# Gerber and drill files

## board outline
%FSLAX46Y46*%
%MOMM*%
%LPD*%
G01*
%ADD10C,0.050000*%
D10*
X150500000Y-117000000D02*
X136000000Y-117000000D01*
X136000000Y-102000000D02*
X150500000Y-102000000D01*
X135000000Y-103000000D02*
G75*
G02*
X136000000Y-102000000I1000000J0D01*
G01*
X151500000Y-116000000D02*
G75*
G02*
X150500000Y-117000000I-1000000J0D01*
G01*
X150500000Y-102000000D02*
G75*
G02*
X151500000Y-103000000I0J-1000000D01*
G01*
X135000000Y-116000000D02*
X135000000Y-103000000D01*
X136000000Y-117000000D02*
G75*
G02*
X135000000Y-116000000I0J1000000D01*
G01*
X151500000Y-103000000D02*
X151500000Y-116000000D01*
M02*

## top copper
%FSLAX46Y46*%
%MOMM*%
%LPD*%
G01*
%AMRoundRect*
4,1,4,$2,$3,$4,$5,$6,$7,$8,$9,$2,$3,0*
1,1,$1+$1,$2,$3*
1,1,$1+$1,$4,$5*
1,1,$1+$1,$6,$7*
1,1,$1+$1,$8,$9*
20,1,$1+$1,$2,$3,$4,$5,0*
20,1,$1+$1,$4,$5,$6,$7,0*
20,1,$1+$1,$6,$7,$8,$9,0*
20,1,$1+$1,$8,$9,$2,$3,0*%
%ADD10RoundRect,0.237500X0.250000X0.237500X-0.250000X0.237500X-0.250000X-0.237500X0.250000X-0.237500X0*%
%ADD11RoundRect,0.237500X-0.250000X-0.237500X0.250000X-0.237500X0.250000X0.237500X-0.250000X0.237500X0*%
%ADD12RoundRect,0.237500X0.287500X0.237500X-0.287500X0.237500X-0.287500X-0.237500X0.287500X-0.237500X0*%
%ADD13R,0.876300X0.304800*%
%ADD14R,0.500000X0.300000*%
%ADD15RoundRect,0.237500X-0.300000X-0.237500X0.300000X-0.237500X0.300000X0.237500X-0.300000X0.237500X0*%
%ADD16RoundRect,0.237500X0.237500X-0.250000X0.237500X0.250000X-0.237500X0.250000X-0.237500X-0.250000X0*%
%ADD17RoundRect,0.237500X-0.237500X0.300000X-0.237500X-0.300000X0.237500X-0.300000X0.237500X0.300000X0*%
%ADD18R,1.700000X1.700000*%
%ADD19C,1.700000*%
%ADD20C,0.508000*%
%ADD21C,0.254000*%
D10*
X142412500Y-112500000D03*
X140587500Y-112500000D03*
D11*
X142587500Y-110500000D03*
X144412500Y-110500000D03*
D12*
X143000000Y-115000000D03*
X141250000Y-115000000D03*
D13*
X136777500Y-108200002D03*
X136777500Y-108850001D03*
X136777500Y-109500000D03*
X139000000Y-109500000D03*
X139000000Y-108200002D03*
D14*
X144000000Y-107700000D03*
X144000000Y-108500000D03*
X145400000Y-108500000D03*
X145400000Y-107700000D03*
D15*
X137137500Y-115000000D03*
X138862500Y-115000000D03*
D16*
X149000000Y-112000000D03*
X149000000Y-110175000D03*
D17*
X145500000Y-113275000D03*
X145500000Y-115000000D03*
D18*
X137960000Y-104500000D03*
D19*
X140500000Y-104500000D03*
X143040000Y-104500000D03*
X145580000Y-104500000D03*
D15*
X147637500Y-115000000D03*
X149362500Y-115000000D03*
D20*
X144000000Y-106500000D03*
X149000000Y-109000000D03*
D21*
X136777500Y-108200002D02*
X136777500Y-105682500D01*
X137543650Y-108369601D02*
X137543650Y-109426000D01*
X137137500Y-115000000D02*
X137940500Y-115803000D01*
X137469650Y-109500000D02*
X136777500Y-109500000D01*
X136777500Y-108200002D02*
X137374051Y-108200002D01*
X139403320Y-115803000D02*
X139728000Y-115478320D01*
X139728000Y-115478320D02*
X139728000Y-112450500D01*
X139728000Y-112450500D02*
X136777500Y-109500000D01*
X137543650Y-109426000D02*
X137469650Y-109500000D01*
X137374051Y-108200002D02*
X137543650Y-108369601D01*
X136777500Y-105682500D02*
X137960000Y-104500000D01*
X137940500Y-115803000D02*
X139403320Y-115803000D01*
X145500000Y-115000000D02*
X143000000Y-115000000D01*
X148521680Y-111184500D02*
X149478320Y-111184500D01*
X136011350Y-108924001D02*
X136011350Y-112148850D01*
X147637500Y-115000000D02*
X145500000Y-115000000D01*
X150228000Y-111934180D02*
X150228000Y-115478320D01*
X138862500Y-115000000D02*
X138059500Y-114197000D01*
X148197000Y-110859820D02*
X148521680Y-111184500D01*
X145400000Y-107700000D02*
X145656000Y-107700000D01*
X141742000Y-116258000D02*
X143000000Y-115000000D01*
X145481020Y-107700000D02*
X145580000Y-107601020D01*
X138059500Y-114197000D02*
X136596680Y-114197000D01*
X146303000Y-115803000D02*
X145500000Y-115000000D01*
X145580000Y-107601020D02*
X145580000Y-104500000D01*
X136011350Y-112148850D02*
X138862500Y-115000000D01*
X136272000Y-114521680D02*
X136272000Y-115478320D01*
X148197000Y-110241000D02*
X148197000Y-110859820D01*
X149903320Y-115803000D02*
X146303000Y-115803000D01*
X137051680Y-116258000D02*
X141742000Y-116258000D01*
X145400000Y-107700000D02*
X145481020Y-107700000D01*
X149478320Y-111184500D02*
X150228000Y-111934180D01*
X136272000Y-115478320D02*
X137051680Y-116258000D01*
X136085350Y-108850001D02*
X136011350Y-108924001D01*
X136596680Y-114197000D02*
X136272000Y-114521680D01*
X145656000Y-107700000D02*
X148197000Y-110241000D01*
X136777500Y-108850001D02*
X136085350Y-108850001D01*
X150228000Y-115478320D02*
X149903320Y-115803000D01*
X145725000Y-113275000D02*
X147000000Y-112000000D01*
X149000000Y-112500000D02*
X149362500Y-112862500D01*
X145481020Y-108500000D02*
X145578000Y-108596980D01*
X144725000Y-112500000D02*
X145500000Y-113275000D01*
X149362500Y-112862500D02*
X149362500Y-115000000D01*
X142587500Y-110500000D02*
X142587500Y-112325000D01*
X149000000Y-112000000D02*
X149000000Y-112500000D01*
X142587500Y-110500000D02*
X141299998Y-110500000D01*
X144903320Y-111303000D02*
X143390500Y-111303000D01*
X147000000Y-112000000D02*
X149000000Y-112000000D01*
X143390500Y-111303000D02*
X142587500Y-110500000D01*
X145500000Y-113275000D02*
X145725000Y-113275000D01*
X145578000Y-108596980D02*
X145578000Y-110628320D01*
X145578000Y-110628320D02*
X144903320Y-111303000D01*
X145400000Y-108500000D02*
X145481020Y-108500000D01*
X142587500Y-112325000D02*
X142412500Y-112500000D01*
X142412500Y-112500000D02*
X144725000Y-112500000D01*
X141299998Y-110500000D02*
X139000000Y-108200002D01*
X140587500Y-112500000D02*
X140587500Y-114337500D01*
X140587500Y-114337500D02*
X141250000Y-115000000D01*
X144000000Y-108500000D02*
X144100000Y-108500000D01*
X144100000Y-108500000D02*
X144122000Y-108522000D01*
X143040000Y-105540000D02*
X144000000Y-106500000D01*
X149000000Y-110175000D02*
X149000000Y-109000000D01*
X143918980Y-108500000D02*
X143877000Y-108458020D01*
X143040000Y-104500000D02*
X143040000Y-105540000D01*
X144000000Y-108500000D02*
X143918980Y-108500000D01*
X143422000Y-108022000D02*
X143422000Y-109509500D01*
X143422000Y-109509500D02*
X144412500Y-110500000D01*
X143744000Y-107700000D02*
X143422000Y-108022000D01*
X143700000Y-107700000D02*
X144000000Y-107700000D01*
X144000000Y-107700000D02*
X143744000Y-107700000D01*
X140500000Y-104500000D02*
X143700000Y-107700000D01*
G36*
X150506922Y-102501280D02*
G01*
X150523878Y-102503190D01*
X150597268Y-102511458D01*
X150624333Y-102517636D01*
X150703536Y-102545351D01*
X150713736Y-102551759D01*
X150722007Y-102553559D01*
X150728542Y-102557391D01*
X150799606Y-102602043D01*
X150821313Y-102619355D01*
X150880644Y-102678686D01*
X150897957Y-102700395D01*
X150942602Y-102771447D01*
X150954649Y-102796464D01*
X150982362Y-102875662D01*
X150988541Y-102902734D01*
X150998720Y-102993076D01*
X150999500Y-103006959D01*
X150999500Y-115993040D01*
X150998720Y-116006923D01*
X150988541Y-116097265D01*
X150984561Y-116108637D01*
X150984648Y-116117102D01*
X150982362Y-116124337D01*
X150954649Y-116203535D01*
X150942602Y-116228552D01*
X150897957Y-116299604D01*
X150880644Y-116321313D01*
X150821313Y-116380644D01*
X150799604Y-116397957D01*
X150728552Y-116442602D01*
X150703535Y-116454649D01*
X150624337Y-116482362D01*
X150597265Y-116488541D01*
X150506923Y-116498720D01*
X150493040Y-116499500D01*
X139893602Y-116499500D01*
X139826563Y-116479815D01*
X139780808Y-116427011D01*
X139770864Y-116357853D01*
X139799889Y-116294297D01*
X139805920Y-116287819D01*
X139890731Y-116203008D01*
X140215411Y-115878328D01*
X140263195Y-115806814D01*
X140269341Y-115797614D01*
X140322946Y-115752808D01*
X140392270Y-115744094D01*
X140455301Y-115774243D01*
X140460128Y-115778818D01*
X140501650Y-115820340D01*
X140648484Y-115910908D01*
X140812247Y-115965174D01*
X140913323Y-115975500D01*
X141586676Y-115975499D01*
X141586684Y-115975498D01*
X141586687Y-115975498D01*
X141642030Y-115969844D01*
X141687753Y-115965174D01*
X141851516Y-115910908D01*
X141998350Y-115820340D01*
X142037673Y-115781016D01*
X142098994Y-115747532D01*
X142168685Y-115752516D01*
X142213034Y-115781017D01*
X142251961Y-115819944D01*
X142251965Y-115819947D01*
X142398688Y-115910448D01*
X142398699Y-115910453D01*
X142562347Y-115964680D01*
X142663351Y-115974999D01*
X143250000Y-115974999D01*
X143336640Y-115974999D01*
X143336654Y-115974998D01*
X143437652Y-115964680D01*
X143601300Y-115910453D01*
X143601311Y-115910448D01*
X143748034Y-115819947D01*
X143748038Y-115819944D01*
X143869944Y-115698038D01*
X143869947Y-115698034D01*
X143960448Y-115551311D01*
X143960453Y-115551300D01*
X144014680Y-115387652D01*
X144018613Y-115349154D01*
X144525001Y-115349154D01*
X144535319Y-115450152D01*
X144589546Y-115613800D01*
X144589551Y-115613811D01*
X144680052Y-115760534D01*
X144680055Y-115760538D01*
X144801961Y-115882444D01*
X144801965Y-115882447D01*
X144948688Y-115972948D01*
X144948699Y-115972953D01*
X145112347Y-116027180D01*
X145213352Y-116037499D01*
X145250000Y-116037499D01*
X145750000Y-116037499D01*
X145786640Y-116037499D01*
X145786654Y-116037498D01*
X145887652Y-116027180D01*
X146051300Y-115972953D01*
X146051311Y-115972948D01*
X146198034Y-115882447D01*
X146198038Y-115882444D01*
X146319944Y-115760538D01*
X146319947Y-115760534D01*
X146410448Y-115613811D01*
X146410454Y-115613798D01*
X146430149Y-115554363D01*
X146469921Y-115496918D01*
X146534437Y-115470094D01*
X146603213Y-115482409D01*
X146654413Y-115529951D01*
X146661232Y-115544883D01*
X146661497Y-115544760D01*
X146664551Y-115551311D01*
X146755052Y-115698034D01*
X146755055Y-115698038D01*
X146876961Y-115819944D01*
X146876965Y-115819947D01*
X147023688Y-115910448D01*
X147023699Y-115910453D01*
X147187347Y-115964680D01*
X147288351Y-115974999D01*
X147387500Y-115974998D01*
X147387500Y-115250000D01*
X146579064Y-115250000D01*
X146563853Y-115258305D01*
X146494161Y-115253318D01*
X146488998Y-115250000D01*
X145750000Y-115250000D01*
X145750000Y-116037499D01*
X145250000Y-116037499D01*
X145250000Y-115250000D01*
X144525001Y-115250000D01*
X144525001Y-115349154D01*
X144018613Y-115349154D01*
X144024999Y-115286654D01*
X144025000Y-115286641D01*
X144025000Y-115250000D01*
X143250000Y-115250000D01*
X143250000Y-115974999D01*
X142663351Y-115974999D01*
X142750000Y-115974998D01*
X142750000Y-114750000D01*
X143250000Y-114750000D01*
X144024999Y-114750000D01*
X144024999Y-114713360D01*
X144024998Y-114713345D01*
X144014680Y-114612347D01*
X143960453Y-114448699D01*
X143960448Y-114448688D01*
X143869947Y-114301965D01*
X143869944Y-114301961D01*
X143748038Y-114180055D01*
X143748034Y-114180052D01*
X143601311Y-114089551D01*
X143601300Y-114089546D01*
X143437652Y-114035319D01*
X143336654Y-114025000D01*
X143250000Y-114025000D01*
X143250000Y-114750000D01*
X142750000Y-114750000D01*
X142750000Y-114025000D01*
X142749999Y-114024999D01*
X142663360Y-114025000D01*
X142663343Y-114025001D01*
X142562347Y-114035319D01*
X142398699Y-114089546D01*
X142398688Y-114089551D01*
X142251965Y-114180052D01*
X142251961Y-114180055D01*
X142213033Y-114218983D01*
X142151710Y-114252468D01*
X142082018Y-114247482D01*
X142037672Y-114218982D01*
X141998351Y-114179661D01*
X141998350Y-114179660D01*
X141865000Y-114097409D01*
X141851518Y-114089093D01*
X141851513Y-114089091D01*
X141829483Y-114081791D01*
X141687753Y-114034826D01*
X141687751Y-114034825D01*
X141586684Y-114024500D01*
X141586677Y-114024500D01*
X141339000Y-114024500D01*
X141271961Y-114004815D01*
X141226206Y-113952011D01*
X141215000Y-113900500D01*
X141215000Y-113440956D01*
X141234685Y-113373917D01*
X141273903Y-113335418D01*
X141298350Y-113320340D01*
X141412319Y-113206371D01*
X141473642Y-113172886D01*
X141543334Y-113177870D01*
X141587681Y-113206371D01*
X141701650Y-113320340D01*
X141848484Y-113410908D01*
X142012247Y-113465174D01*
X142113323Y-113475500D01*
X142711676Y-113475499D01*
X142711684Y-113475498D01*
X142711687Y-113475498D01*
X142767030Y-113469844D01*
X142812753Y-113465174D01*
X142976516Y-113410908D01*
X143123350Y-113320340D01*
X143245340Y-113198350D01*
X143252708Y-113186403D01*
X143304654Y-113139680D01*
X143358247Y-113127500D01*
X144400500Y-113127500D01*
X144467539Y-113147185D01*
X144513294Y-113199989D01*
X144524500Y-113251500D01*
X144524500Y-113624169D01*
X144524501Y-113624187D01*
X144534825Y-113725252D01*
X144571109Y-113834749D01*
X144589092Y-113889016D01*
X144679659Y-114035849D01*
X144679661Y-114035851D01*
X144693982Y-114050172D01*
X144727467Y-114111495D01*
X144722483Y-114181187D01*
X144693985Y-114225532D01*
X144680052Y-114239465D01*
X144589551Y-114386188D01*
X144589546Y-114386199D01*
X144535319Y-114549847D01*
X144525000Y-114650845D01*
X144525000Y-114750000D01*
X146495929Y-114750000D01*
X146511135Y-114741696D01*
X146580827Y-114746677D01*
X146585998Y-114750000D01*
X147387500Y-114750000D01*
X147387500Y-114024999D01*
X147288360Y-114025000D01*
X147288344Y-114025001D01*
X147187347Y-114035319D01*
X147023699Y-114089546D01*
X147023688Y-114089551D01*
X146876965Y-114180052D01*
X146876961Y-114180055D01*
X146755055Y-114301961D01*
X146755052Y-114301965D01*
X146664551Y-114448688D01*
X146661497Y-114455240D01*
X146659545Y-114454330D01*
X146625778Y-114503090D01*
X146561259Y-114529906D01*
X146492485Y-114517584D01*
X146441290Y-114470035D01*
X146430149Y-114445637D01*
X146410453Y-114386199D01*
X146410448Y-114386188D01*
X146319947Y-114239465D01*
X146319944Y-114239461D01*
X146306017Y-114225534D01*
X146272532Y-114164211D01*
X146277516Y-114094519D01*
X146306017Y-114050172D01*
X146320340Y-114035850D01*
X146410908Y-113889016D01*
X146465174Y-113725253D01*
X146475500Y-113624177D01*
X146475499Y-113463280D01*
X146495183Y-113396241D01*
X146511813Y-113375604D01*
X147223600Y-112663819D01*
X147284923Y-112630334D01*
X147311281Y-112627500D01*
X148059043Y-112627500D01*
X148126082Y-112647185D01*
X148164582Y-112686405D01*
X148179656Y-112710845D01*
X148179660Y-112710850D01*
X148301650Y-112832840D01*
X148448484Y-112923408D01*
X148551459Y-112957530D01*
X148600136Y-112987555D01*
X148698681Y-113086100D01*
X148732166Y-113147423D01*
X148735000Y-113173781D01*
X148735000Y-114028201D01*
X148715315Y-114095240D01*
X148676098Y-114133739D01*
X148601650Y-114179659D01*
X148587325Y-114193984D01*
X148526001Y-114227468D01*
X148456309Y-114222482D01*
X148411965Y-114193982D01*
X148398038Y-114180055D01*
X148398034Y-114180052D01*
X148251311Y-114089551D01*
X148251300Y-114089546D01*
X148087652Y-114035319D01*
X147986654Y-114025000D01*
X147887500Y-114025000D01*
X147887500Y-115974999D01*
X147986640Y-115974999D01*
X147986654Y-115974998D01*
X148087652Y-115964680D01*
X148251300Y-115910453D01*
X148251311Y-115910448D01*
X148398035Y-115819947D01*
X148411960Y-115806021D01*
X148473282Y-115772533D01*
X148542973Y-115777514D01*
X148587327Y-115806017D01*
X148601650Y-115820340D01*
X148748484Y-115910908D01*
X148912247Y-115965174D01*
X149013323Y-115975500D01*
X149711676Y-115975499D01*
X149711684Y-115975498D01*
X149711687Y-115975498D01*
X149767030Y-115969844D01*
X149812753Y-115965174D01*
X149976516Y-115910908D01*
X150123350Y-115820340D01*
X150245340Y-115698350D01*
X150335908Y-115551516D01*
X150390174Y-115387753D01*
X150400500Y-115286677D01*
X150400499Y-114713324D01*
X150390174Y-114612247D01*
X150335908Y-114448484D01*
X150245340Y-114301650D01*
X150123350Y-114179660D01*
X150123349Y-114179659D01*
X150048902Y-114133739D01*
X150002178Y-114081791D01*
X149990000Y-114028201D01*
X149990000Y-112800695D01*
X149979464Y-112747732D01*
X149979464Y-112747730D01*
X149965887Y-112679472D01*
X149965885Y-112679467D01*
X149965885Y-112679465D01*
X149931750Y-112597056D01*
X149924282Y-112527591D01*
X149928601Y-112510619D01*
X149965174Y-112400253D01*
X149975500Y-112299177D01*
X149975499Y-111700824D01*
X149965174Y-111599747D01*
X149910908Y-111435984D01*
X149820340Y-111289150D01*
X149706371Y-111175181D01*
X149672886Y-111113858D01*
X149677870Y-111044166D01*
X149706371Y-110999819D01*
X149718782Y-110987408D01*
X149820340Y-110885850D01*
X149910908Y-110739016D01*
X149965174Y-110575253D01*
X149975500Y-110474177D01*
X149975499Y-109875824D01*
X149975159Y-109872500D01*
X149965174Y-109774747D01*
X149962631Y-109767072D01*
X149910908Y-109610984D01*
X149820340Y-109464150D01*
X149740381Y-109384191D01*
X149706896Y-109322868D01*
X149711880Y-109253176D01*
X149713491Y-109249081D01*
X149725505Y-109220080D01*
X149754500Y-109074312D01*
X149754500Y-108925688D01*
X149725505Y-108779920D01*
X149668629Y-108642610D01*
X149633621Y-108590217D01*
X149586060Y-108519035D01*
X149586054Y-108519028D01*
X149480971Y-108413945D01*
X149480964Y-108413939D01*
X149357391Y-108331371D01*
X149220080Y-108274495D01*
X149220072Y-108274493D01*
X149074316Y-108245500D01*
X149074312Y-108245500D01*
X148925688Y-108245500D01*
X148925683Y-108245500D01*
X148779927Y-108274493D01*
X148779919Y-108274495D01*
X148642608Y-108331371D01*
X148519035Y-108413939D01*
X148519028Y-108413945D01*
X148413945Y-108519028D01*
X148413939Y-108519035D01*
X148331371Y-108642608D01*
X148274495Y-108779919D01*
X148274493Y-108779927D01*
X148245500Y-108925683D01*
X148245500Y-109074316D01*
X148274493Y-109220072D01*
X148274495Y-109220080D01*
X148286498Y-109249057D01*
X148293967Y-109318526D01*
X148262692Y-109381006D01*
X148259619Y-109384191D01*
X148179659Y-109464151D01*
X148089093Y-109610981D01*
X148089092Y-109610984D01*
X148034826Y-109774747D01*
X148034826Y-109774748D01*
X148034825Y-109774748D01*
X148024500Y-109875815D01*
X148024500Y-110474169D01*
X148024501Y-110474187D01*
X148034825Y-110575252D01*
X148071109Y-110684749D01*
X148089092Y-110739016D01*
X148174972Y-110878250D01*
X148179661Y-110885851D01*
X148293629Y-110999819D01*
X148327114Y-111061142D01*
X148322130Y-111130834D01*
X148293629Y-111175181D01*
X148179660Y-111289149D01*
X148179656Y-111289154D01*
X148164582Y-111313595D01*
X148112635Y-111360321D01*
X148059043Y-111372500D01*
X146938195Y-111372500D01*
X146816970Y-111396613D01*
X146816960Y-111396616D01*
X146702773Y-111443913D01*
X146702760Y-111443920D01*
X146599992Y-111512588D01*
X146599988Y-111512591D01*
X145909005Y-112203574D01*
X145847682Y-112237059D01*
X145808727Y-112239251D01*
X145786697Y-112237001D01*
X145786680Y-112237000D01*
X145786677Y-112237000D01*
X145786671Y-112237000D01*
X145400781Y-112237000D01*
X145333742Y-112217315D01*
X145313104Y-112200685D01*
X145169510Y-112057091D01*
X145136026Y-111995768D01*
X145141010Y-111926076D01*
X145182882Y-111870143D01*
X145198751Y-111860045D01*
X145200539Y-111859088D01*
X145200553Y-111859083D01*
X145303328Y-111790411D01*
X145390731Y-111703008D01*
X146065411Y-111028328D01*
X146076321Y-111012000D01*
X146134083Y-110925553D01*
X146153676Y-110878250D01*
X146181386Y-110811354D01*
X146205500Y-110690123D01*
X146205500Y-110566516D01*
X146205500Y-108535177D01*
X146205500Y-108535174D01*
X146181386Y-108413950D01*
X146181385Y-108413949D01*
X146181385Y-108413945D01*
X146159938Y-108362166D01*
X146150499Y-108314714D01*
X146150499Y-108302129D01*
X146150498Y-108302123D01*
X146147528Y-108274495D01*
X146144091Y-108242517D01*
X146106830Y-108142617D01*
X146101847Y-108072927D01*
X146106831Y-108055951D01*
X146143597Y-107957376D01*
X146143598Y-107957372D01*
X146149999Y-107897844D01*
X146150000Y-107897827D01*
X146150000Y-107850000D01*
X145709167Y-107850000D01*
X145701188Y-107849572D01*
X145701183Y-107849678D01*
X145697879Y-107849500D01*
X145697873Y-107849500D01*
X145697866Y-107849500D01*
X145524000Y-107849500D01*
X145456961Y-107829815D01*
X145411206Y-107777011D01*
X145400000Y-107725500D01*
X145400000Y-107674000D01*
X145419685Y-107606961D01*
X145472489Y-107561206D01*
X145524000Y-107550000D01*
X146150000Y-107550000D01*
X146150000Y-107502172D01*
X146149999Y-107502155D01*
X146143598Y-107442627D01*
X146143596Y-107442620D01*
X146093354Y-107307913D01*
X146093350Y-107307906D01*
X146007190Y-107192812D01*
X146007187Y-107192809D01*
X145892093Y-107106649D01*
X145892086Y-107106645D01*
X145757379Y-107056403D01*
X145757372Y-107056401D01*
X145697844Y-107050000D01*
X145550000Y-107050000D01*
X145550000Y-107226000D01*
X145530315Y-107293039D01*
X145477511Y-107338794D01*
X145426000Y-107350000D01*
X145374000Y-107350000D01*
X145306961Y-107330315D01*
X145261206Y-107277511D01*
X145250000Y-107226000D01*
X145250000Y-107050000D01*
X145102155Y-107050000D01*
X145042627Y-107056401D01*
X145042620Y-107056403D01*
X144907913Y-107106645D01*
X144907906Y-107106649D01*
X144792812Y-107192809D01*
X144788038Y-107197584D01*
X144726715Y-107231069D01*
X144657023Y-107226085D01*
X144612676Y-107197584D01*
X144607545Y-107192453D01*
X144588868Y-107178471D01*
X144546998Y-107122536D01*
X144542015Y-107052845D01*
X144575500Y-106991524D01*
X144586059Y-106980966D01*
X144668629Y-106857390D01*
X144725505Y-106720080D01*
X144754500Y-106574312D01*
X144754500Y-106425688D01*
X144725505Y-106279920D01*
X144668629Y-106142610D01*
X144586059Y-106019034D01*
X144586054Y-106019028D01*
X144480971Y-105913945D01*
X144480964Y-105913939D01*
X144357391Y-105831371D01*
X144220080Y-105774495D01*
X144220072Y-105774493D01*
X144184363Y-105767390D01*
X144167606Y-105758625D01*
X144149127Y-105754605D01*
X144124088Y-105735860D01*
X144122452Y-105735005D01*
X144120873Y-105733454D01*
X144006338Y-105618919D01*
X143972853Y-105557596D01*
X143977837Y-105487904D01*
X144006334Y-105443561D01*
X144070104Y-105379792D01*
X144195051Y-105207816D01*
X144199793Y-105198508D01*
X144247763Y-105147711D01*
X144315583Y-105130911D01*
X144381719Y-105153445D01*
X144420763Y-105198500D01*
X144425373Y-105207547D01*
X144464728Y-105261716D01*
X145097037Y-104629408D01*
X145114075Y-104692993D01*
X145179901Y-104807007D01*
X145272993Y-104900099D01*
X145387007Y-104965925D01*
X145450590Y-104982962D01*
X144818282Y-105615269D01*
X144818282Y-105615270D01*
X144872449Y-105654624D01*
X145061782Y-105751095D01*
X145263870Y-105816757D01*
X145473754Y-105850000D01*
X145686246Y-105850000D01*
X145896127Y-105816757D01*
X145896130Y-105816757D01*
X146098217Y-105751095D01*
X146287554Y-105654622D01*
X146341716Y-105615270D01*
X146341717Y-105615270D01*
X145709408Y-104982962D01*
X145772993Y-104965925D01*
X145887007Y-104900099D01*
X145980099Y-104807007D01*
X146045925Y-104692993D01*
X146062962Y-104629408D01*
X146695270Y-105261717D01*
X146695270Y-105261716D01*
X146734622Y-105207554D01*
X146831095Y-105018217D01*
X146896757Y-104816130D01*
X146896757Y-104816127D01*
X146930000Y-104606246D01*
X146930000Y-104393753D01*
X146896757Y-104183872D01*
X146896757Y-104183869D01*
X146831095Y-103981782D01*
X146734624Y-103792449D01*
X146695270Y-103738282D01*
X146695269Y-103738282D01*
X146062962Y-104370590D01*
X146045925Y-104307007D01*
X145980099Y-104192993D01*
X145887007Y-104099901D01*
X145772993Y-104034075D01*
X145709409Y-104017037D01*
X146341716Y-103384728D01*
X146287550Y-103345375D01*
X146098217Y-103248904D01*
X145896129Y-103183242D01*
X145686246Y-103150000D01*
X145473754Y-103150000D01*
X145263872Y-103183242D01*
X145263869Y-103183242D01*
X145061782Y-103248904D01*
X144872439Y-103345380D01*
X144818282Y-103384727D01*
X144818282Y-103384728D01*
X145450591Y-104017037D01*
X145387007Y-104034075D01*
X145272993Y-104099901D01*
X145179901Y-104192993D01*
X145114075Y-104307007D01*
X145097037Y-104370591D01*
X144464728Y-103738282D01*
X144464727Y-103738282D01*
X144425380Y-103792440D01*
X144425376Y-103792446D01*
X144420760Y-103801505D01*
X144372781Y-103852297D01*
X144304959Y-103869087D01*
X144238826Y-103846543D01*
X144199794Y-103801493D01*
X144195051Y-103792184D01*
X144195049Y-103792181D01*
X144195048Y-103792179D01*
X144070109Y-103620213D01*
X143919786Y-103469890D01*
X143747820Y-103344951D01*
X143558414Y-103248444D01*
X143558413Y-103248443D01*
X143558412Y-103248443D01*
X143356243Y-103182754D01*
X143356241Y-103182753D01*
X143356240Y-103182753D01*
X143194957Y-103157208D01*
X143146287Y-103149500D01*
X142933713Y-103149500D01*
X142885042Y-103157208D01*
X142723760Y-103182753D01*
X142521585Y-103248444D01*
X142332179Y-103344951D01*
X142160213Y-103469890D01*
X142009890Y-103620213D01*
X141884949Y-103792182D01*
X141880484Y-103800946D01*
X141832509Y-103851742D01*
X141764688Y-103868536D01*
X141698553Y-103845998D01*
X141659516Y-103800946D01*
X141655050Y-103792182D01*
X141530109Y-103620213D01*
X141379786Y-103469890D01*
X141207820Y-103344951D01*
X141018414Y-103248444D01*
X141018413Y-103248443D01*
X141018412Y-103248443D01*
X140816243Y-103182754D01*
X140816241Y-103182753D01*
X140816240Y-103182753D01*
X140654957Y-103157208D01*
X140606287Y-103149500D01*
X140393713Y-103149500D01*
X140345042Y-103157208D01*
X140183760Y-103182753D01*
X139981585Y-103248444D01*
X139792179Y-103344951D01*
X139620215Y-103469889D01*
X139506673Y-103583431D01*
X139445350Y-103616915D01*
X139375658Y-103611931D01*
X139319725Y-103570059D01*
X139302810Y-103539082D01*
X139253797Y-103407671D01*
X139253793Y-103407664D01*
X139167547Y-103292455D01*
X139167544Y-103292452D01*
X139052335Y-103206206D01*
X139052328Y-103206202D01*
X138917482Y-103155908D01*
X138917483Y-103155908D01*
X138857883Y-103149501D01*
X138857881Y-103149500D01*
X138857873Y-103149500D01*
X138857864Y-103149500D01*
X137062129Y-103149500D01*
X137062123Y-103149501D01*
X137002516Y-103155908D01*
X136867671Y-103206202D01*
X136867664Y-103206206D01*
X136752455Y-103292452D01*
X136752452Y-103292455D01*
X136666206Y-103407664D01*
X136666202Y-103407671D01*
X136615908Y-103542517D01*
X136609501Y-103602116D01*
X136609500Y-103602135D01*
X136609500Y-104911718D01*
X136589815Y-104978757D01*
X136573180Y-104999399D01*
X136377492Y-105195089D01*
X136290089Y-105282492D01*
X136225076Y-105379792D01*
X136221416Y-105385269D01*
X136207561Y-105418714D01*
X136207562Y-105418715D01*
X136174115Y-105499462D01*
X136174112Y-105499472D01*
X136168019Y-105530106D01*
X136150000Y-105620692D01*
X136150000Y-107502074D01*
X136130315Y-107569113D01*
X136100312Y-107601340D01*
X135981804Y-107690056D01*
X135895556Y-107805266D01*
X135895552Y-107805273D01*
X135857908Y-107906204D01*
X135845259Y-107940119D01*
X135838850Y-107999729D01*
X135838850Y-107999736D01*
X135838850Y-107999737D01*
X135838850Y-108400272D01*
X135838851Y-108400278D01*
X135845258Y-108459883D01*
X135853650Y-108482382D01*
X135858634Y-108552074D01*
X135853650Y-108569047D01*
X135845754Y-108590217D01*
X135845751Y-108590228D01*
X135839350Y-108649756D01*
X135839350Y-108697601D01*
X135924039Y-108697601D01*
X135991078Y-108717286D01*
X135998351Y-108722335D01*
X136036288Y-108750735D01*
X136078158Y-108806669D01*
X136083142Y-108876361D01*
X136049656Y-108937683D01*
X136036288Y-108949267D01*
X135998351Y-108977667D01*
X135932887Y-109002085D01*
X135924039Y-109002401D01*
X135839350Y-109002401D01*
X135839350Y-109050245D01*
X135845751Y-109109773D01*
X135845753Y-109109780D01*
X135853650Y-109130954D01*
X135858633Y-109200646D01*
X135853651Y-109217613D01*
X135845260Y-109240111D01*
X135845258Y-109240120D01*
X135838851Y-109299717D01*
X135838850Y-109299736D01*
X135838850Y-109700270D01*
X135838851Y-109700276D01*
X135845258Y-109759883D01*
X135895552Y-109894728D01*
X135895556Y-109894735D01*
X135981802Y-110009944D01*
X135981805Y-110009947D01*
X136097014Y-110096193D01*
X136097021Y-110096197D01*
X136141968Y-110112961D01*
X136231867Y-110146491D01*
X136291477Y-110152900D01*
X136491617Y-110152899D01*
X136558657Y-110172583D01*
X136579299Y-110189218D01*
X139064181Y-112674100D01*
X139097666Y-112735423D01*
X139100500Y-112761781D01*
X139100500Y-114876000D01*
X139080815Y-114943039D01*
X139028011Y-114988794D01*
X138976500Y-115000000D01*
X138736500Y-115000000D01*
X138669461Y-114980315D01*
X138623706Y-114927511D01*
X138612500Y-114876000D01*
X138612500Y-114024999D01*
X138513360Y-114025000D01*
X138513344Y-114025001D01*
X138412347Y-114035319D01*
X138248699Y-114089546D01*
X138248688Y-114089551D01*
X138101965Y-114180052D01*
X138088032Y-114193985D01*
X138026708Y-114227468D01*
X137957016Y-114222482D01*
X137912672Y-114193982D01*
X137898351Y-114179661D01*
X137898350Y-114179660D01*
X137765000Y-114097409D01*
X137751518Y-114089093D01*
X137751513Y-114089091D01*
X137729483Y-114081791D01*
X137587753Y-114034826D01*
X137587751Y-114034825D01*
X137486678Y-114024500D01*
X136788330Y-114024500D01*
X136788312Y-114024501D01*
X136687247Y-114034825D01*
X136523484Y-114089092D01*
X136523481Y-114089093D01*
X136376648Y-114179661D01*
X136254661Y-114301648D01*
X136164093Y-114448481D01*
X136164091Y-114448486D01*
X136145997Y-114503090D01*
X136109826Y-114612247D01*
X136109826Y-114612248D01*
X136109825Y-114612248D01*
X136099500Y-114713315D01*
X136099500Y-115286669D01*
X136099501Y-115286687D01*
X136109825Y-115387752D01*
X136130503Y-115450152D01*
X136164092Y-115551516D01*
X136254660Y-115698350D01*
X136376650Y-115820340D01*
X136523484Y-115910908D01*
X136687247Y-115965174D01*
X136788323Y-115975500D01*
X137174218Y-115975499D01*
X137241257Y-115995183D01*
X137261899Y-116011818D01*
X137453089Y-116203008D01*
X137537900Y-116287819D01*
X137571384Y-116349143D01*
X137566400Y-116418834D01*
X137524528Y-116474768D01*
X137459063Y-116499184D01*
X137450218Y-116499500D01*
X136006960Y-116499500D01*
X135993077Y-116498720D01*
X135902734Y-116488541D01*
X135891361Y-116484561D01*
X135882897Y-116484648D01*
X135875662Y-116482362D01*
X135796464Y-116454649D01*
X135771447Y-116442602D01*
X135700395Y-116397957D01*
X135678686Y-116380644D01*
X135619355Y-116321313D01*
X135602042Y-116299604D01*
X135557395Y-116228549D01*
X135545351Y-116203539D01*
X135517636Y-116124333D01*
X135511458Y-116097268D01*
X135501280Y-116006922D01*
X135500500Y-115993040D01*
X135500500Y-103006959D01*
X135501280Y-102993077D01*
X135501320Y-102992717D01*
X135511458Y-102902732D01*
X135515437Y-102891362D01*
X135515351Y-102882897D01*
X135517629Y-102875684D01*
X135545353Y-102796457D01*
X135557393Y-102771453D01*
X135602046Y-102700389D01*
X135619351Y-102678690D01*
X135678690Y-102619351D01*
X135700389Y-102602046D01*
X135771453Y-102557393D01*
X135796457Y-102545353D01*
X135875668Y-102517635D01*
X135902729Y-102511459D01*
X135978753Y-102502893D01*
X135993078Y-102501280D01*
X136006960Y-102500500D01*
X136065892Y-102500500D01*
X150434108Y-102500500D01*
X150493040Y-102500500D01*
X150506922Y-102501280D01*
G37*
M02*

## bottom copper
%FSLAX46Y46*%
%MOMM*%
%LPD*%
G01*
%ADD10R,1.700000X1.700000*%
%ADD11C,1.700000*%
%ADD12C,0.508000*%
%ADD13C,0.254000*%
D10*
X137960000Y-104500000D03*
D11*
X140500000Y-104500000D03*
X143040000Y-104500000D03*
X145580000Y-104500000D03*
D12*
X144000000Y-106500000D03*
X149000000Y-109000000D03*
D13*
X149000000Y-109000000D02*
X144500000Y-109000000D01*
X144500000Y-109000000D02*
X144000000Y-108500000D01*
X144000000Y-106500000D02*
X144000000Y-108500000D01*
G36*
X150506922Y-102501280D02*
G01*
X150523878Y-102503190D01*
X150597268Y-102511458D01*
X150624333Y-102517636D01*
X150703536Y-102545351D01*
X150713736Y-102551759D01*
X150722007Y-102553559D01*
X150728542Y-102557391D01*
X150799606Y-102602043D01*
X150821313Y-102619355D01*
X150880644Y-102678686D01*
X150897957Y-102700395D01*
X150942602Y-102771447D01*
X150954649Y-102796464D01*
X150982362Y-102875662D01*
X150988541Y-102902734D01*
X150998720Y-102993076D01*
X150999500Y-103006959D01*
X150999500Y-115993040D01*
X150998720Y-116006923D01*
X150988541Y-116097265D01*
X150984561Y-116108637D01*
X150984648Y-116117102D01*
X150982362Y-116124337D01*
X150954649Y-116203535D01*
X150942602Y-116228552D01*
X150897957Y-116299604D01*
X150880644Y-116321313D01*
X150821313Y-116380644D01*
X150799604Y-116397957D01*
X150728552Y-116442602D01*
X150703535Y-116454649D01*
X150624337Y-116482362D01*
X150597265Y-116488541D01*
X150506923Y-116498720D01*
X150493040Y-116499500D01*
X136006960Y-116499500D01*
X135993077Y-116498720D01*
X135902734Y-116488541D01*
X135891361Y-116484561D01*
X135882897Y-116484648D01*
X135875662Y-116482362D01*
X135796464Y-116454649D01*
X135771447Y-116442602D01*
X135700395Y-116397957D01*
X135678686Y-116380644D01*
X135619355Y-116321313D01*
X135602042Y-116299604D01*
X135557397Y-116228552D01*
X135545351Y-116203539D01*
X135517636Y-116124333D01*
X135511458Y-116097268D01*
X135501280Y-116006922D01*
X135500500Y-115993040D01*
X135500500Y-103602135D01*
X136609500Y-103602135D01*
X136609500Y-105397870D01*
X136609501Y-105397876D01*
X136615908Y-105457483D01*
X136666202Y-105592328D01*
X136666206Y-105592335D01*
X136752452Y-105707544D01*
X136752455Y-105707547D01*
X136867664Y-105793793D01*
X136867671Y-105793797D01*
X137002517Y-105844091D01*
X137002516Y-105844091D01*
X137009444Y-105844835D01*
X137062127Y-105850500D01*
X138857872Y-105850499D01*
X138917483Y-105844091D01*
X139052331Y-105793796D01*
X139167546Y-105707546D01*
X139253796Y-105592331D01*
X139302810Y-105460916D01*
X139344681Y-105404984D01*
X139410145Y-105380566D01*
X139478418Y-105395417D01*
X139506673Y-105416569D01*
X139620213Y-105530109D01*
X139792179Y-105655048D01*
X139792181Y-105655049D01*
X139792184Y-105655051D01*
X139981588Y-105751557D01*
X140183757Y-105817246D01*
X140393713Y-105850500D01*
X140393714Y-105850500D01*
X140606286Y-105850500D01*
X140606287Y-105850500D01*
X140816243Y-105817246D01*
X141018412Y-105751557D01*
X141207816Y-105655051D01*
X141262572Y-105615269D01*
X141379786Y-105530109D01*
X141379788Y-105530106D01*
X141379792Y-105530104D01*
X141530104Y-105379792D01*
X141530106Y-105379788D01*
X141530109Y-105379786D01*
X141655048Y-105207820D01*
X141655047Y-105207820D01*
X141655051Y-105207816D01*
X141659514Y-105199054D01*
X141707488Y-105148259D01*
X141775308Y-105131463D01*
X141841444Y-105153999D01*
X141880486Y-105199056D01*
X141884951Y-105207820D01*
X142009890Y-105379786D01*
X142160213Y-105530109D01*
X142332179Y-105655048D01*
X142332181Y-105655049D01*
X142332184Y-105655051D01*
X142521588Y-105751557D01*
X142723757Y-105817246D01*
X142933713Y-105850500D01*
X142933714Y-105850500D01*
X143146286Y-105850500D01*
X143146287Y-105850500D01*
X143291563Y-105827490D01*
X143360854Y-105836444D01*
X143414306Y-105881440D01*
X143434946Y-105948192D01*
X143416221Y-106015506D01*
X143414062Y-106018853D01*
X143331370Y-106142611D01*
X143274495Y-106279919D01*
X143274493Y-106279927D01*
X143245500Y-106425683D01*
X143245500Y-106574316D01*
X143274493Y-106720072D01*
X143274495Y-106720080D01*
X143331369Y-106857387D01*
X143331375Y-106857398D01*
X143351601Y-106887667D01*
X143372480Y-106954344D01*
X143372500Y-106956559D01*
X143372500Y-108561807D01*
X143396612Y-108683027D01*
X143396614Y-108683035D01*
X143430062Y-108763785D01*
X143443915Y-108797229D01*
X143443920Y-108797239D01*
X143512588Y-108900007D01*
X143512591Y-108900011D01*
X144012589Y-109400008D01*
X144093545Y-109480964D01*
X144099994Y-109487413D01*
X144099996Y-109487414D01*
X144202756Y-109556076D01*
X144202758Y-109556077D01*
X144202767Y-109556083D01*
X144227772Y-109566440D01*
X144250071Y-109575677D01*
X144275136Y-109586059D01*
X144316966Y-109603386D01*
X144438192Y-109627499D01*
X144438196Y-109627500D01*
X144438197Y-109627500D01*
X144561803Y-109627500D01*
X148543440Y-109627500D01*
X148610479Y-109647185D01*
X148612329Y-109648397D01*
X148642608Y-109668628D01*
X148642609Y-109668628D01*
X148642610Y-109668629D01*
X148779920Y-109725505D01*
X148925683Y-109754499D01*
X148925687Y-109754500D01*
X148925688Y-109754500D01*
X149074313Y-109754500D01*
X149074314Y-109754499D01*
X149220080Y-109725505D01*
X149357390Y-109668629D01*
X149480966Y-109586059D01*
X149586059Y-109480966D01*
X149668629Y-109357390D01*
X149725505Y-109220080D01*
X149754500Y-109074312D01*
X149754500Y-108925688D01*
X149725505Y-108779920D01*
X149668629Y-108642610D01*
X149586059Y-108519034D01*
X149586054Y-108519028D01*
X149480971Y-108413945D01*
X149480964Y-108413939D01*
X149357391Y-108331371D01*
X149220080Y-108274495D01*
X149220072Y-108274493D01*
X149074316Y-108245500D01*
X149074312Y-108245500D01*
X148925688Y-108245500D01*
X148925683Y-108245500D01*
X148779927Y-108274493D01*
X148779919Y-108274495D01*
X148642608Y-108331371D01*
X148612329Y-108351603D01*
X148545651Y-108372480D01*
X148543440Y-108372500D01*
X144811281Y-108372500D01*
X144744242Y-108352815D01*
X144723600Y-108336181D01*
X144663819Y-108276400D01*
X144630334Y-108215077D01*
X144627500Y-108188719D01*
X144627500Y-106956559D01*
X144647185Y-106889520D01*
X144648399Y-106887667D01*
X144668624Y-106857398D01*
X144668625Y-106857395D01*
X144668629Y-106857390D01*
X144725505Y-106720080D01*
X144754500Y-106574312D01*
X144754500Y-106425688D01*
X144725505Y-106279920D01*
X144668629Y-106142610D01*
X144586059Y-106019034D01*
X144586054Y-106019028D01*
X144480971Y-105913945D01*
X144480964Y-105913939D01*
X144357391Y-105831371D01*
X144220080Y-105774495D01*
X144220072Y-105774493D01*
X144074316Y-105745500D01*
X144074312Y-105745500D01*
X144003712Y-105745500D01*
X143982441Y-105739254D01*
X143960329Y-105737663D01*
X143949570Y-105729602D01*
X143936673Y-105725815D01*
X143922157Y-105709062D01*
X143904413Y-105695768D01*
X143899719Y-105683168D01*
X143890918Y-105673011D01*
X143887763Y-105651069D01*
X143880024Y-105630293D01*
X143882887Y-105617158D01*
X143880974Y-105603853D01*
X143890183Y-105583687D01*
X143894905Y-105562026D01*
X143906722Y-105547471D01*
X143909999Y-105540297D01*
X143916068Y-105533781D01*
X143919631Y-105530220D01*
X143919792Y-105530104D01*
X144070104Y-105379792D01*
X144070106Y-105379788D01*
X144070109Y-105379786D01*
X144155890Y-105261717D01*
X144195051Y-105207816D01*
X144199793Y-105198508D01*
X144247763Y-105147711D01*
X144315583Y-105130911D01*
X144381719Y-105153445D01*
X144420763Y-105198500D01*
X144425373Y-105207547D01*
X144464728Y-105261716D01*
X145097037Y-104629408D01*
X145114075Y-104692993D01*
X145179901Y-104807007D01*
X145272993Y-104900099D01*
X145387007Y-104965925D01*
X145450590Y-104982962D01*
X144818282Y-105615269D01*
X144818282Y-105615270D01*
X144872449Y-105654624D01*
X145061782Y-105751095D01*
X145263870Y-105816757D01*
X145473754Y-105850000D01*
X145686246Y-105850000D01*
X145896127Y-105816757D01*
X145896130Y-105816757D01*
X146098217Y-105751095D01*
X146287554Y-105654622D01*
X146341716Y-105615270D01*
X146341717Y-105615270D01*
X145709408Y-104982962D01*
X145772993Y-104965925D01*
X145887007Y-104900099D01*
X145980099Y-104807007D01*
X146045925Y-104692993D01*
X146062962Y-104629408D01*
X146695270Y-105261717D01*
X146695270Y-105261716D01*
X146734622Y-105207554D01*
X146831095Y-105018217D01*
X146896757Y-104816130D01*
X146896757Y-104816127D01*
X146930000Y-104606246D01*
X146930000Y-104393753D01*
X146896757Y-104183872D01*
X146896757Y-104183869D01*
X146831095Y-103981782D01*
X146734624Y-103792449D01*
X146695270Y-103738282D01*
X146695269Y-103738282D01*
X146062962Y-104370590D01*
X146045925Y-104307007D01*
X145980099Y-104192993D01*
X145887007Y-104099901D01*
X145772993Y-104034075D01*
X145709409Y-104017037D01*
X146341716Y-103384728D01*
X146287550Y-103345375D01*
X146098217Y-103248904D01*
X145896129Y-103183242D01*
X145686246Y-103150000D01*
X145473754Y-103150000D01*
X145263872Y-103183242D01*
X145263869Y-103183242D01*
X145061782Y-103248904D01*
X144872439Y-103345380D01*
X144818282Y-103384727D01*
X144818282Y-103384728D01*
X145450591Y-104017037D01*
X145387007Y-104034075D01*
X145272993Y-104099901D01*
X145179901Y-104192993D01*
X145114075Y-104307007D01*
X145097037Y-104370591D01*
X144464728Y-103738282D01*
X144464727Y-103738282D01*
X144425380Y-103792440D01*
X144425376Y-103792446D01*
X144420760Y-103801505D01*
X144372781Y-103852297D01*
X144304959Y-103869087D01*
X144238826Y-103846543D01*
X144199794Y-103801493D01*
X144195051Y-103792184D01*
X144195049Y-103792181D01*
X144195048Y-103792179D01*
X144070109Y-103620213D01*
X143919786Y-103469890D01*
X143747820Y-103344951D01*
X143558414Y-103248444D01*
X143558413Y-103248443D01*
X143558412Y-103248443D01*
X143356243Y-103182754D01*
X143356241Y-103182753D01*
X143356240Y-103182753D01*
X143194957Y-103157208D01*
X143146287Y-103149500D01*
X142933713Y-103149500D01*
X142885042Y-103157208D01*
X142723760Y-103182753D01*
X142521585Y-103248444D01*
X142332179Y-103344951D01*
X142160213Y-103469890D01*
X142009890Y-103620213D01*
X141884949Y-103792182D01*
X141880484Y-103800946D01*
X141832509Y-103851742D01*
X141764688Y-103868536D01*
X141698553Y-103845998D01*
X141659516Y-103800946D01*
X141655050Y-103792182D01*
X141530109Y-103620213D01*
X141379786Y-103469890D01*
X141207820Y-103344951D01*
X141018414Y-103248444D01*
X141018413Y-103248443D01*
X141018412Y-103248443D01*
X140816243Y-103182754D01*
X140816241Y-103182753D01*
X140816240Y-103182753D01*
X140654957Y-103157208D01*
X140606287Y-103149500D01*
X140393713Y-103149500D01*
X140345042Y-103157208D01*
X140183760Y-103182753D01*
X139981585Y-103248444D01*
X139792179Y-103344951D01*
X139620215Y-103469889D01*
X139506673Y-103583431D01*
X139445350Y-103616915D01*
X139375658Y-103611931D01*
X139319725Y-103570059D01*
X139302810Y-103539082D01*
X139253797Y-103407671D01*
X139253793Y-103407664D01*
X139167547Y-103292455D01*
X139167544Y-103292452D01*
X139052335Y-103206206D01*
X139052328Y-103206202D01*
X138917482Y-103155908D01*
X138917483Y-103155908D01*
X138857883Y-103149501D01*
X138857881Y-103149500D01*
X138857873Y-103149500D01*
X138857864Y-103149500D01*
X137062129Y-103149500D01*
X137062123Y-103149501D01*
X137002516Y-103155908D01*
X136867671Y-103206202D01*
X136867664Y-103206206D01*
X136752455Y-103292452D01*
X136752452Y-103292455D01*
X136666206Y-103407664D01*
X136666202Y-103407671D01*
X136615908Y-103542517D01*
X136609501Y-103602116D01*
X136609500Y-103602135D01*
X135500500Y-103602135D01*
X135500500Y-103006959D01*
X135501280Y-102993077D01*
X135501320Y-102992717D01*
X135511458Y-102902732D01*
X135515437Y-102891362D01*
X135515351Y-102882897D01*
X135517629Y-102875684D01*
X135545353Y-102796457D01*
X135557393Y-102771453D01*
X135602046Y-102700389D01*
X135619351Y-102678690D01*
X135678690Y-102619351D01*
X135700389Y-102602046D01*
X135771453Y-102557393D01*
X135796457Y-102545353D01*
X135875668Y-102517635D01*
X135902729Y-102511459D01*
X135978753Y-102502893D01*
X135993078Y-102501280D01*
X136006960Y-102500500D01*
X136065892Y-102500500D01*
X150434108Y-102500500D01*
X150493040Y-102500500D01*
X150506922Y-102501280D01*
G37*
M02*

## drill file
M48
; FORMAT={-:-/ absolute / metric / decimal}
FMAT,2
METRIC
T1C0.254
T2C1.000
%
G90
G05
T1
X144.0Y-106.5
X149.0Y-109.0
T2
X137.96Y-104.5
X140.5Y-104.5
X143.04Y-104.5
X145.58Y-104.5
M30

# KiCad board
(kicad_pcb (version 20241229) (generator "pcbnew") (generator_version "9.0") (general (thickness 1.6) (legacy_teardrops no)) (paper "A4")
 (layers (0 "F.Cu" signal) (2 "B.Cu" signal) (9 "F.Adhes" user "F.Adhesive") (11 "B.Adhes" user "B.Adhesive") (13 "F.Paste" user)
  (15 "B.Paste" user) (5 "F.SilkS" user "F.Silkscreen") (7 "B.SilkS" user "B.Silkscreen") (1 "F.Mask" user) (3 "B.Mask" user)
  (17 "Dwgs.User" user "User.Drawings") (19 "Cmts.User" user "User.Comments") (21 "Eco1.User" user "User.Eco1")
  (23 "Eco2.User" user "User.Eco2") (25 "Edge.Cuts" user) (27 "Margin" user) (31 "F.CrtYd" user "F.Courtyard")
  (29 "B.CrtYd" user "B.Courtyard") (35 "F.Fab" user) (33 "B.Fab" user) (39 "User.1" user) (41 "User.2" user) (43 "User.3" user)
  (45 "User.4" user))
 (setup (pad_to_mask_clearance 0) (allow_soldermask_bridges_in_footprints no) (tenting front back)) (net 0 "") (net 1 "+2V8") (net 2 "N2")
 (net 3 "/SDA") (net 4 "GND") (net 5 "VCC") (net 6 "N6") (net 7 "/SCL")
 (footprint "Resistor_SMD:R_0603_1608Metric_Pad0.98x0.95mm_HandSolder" (layer "F.Cu") (at 141.5 112.5 180)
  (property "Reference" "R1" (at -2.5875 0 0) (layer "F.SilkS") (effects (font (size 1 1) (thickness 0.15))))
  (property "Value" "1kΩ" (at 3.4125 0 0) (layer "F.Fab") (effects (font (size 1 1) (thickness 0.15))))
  (pad "1" smd roundrect (at -0.9125 0 180) (size 0.975 0.95) (layers "F.Cu" "F.Mask" "F.Paste") (roundrect_rratio 0.25) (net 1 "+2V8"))
  (pad "2" smd roundrect (at 0.9125 0 180) (size 0.975 0.95) (layers "F.Cu" "F.Mask" "F.Paste") (roundrect_rratio 0.25) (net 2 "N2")))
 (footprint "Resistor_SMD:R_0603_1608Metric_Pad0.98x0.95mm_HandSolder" (layer "F.Cu") (at 143.5 110.5)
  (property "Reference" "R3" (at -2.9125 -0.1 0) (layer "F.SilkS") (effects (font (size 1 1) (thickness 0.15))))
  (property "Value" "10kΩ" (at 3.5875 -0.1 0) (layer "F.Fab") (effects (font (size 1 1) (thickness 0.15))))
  (pad "1" smd roundrect (at -0.9125 0) (size 0.975 0.95) (layers "F.Cu" "F.Mask" "F.Paste") (roundrect_rratio 0.25) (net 1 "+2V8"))
  (pad "2" smd roundrect (at 0.9125 0) (size 0.975 0.95) (layers "F.Cu" "F.Mask" "F.Paste") (roundrect_rratio 0.25) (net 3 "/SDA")))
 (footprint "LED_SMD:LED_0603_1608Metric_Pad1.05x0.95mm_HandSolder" (layer "F.Cu") (at 142.125 115 180)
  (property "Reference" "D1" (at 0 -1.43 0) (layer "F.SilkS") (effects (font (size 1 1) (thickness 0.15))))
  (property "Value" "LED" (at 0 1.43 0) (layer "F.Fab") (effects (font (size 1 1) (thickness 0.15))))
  (pad "1" smd roundrect (at -0.875 0 180) (size 1.05 0.95) (layers "F.Cu" "F.Mask" "F.Paste") (roundrect_rratio 0.25) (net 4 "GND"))
  (pad "2" smd roundrect (at 0.875 0 180) (size 1.05 0.95) (layers "F.Cu" "F.Mask" "F.Paste") (roundrect_rratio 0.25) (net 2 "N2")))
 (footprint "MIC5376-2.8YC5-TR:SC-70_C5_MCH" (layer "F.Cu") (at 137.88875 108.850001)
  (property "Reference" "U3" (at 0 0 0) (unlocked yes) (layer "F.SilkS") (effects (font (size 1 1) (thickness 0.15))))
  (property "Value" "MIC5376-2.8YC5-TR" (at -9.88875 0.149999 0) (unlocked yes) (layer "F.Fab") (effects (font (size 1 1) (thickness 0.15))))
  (pad "1" smd rect (at -1.11125 -0.649999) (size 0.8763 0.3048) (layers "F.Cu" "F.Mask" "F.Paste") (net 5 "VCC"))
  (pad "2" smd rect (at -1.11125 0) (size 0.8763 0.3048) (layers "F.Cu" "F.Mask" "F.Paste") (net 4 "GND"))
  (pad "3" smd rect (at -1.11125 0.649999) (size 0.8763 0.3048) (layers "F.Cu" "F.Mask" "F.Paste") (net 5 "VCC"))
  (pad "4" smd rect (at 1.11125 0.649999) (size 0.8763 0.3048) (layers "F.Cu" "F.Mask" "F.Paste") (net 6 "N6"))
  (pad "5" smd rect (at 1.11125 -0.649999) (size 0.8763 0.3048) (layers "F.Cu" "F.Mask" "F.Paste") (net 1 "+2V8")))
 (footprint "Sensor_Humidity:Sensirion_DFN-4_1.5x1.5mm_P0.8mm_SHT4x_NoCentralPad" (layer "F.Cu") (at 144.7 108.1)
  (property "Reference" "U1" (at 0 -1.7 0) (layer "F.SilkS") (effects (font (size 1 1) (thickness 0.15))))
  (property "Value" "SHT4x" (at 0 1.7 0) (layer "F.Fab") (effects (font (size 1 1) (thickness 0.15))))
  (pad "1" smd rect (at -0.7 -0.4) (size 0.5 0.3) (layers "F.Cu" "F.Mask" "F.Paste") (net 3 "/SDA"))
  (pad "2" smd rect (at -0.7 0.4) (size 0.5 0.3) (layers "F.Cu" "F.Mask" "F.Paste") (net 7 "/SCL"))
  (pad "3" smd rect (at 0.7 0.4) (size 0.5 0.3) (layers "F.Cu" "F.Mask" "F.Paste") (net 1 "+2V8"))
  (pad "4" smd rect (at 0.7 -0.4) (size 0.5 0.3) (layers "F.Cu" "F.Mask" "F.Paste") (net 4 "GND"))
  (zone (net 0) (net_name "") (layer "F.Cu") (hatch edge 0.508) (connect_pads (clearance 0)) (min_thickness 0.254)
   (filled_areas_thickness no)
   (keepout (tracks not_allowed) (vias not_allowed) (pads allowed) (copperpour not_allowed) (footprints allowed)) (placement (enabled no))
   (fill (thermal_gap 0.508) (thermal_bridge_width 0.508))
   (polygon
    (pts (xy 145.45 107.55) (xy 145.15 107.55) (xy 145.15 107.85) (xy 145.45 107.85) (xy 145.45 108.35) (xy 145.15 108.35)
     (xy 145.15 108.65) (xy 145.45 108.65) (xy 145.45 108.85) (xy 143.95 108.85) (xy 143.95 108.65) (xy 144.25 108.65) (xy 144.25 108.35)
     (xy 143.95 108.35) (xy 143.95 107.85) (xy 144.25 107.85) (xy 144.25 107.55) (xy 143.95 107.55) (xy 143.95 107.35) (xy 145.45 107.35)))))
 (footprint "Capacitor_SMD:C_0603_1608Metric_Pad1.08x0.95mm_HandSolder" (layer "F.Cu") (at 138 115)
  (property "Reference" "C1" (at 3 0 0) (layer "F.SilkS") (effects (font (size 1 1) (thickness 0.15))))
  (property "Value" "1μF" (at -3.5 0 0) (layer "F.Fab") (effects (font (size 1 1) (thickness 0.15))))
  (pad "1" smd roundrect (at -0.8625 0) (size 1.075 0.95) (layers "F.Cu" "F.Mask" "F.Paste") (roundrect_rratio 0.25) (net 5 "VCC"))
  (pad "2" smd roundrect (at 0.8625 0) (size 1.075 0.95) (layers "F.Cu" "F.Mask" "F.Paste") (roundrect_rratio 0.25) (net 4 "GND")))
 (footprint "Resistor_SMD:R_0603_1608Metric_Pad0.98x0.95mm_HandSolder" (layer "F.Cu") (at 149 111.0875 90)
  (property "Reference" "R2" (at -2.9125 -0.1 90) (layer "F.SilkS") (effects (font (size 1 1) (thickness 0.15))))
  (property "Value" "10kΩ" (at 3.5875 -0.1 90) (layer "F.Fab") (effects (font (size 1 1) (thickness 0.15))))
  (pad "1" smd roundrect (at -0.9125 0 90) (size 0.975 0.95) (layers "F.Cu" "F.Mask" "F.Paste") (roundrect_rratio 0.25) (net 1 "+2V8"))
  (pad "2" smd roundrect (at 0.9125 0 90) (size 0.975 0.95) (layers "F.Cu" "F.Mask" "F.Paste") (roundrect_rratio 0.25) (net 7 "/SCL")))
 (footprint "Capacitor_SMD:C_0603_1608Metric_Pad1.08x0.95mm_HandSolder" (layer "F.Cu") (at 145.5 114.1375 -90)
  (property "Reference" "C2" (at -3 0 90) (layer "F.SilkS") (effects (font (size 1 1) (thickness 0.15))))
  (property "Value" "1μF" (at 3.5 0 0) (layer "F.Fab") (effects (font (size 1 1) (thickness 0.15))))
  (pad "1" smd roundrect (at -0.8625 0 270) (size 1.075 0.95) (layers "F.Cu" "F.Mask" "F.Paste") (roundrect_rratio 0.25) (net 1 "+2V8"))
  (pad "2" smd roundrect (at 0.8625 0 270) (size 1.075 0.95) (layers "F.Cu" "F.Mask" "F.Paste") (roundrect_rratio 0.25) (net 4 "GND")))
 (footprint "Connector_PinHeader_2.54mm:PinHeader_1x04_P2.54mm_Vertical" (layer "F.Cu") (at 137.96 104.5 90)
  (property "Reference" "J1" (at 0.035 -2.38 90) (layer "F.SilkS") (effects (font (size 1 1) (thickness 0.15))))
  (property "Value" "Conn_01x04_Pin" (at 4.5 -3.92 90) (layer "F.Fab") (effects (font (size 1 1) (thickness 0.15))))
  (pad "1" thru_hole rect (at 0 0 90) (size 1.7 1.7) (drill 1) (layers "*.Cu" "*.Mask") (remove_unused_layers no) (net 5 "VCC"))
  (pad "2" thru_hole circle (at 0 2.54 90) (size 1.7 1.7) (drill 1) (layers "*.Cu" "*.Mask") (remove_unused_layers no) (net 3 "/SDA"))
  (pad "3" thru_hole circle (at 0 5.08 90) (size 1.7 1.7) (drill 1) (layers "*.Cu" "*.Mask") (remove_unused_layers no) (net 7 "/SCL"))
  (pad "4" thru_hole circle (at 0 7.62 90) (size 1.7 1.7) (drill 1) (layers "*.Cu" "*.Mask") (remove_unused_layers no) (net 4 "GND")))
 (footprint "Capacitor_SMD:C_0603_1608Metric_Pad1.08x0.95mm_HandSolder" (layer "F.Cu") (at 148.5 115)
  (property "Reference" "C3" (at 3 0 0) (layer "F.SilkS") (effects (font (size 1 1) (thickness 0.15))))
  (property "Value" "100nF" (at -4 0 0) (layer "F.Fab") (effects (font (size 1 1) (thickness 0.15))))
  (pad "1" smd roundrect (at -0.8625 0) (size 1.075 0.95) (layers "F.Cu" "F.Mask" "F.Paste") (roundrect_rratio 0.25) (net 4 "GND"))
  (pad "2" smd roundrect (at 0.8625 0) (size 1.075 0.95) (layers "F.Cu" "F.Mask" "F.Paste") (roundrect_rratio 0.25) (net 1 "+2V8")))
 (gr_line (start 150.5 117) (end 136 117) (stroke (width 0.05) (type default)) (layer "Edge.Cuts"))
 (gr_line (start 136 102) (end 150.5 102) (stroke (width 0.05) (type default)) (layer "Edge.Cuts"))
 (gr_arc (start 135 103) (mid 135.292893 102.292893) (end 136 102) (stroke (width 0.05) (type default)) (layer "Edge.Cuts"))
 (gr_arc (start 151.5 116) (mid 151.207107 116.707107) (end 150.5 117) (stroke (width 0.05) (type default)) (layer "Edge.Cuts"))
 (gr_arc (start 150.5 102) (mid 151.207107 102.292893) (end 151.5 103) (stroke (width 0.05) (type default)) (layer "Edge.Cuts"))
 (gr_line (start 135 116) (end 135 103) (stroke (width 0.05) (type default)) (layer "Edge.Cuts"))
 (gr_arc (start 136 117) (mid 135.292893 116.707107) (end 135 116) (stroke (width 0.05) (type default)) (layer "Edge.Cuts"))
 (gr_line (start 151.5 103) (end 151.5 116) (stroke (width 0.05) (type default)) (layer "Edge.Cuts"))
 (segment (start 136.7775 108.200002) (end 136.7775 105.6825) (width 0.254) (layer "F.Cu") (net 5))
 (segment (start 137.54365 108.369601) (end 137.54365 109.426) (width 0.254) (layer "F.Cu") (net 5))
 (segment (start 137.1375 115) (end 137.9405 115.803) (width 0.254) (layer "F.Cu") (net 5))
 (segment (start 137.46965 109.5) (end 136.7775 109.5) (width 0.254) (layer "F.Cu") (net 5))
 (segment (start 136.7775 108.200002) (end 137.374051 108.200002) (width 0.254) (layer "F.Cu") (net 5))
 (segment (start 139.40332 115.803) (end 139.728 115.47832) (width 0.254) (layer "F.Cu") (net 5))
 (segment (start 139.728 115.47832) (end 139.728 112.4505) (width 0.254) (layer "F.Cu") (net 5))
 (segment (start 139.728 112.4505) (end 136.7775 109.5) (width 0.254) (layer "F.Cu") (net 5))
 (segment (start 137.54365 109.426) (end 137.46965 109.5) (width 0.254) (layer "F.Cu") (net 5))
 (segment (start 137.374051 108.200002) (end 137.54365 108.369601) (width 0.254) (layer "F.Cu") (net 5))
 (segment (start 136.7775 105.6825) (end 137.96 104.5) (width 0.254) (layer "F.Cu") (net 5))
 (segment (start 137.9405 115.803) (end 139.40332 115.803) (width 0.254) (layer "F.Cu") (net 5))
 (segment (start 145.5 115) (end 143 115) (width 0.254) (layer "F.Cu") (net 4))
 (segment (start 148.52168 111.1845) (end 149.47832 111.1845) (width 0.254) (layer "F.Cu") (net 4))
 (segment (start 136.01135 108.924001) (end 136.01135 112.14885) (width 0.254) (layer "F.Cu") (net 4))
 (segment (start 147.6375 115) (end 145.5 115) (width 0.254) (layer "F.Cu") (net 4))
 (segment (start 150.228 111.93418) (end 150.228 115.47832) (width 0.254) (layer "F.Cu") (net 4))
 (segment (start 138.8625 115) (end 138.0595 114.197) (width 0.254) (layer "F.Cu") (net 4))
 (segment (start 148.197 110.85982) (end 148.52168 111.1845) (width 0.254) (layer "F.Cu") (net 4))
 (segment (start 145.4 107.7) (end 145.656 107.7) (width 0.254) (layer "F.Cu") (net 4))
 (segment (start 141.742 116.258) (end 143 115) (width 0.254) (layer "F.Cu") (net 4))
 (segment (start 145.48102 107.7) (end 145.58 107.60102) (width 0.254) (layer "F.Cu") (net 4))
 (segment (start 138.0595 114.197) (end 136.59668 114.197) (width 0.254) (layer "F.Cu") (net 4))
 (segment (start 146.303 115.803) (end 145.5 115) (width 0.254) (layer "F.Cu") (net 4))
 (segment (start 145.58 107.60102) (end 145.58 104.5) (width 0.254) (layer "F.Cu") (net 4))
 (segment (start 136.01135 112.14885) (end 138.8625 115) (width 0.254) (layer "F.Cu") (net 4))
 (segment (start 136.272 114.52168) (end 136.272 115.47832) (width 0.254) (layer "F.Cu") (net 4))
 (segment (start 148.197 110.241) (end 148.197 110.85982) (width 0.254) (layer "F.Cu") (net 4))
 (segment (start 149.90332 115.803) (end 146.303 115.803) (width 0.254) (layer "F.Cu") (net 4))
 (segment (start 137.05168 116.258) (end 141.742 116.258) (width 0.254) (layer "F.Cu") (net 4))
 (segment (start 145.4 107.7) (end 145.48102 107.7) (width 0.254) (layer "F.Cu") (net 4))
 (segment (start 149.47832 111.1845) (end 150.228 111.93418) (width 0.254) (layer "F.Cu") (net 4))
 (segment (start 136.272 115.47832) (end 137.05168 116.258) (width 0.254) (layer "F.Cu") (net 4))
 (segment (start 136.08535 108.850001) (end 136.01135 108.924001) (width 0.254) (layer "F.Cu") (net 4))
 (segment (start 136.59668 114.197) (end 136.272 114.52168) (width 0.254) (layer "F.Cu") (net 4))
 (segment (start 145.656 107.7) (end 148.197 110.241) (width 0.254) (layer "F.Cu") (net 4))
 (segment (start 136.7775 108.850001) (end 136.08535 108.850001) (width 0.254) (layer "F.Cu") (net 4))
 (segment (start 150.228 115.47832) (end 149.90332 115.803) (width 0.254) (layer "F.Cu") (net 4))
 (segment (start 145.725 113.275) (end 147 112) (width 0.254) (layer "F.Cu") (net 1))
 (segment (start 149 112.5) (end 149.3625 112.8625) (width 0.254) (layer "F.Cu") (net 1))
 (segment (start 145.48102 108.5) (end 145.578 108.59698) (width 0.254) (layer "F.Cu") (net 1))
 (segment (start 144.725 112.5) (end 145.5 113.275) (width 0.254) (layer "F.Cu") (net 1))
 (segment (start 149.3625 112.8625) (end 149.3625 115) (width 0.254) (layer "F.Cu") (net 1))
 (segment (start 142.5875 110.5) (end 142.5875 112.325) (width 0.254) (layer "F.Cu") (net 1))
 (segment (start 149 112) (end 149 112.5) (width 0.254) (layer "F.Cu") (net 1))
 (segment (start 142.5875 110.5) (end 141.299998 110.5) (width 0.254) (layer "F.Cu") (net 1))
 (segment (start 144.90332 111.303) (end 143.3905 111.303) (width 0.254) (layer "F.Cu") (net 1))
 (segment (start 147 112) (end 149 112) (width 0.254) (layer "F.Cu") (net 1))
 (segment (start 143.3905 111.303) (end 142.5875 110.5) (width 0.254) (layer "F.Cu") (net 1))
 (segment (start 145.5 113.275) (end 145.725 113.275) (width 0.254) (layer "F.Cu") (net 1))
 (segment (start 145.578 108.59698) (end 145.578 110.62832) (width 0.254) (layer "F.Cu") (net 1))
 (segment (start 145.578 110.62832) (end 144.90332 111.303) (width 0.254) (layer "F.Cu") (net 1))
 (segment (start 145.4 108.5) (end 145.48102 108.5) (width 0.254) (layer "F.Cu") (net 1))
 (segment (start 142.5875 112.325) (end 142.4125 112.5) (width 0.254) (layer "F.Cu") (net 1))
 (segment (start 142.4125 112.5) (end 144.725 112.5) (width 0.254) (layer "F.Cu") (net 1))
 (segment (start 141.299998 110.5) (end 139 108.200002) (width 0.254) (layer "F.Cu") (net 1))
 (segment (start 140.5875 112.5) (end 140.5875 114.3375) (width 0.254) (layer "F.Cu") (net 2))
 (segment (start 140.5875 114.3375) (end 141.25 115) (width 0.254) (layer "F.Cu") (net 2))
 (segment (start 144 108.5) (end 144.1 108.5) (width 0.254) (layer "F.Cu") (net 7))
 (segment (start 144.1 108.5) (end 144.122 108.522) (width 0.254) (layer "F.Cu") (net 7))
 (segment (start 143.04 105.54) (end 144 106.5) (width 0.254) (layer "F.Cu") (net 7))
 (segment (start 149 110.175) (end 149 109) (width 0.254) (layer "F.Cu") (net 7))
 (segment (start 143.91898 108.5) (end 143.877 108.45802) (width 0.254) (layer "F.Cu") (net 7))
 (segment (start 143.04 104.5) (end 143.04 105.54) (width 0.254) (layer "F.Cu") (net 7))
 (segment (start 144 108.5) (end 143.91898 108.5) (width 0.254) (layer "F.Cu") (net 7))
 (via (at 144 106.5) (size 0.508) (drill 0.254) (layers "F.Cu" "B.Cu") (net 7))
 (via (at 149 109) (size 0.508) (drill 0.254) (layers "F.Cu" "B.Cu") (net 7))
 (segment (start 149 109) (end 144.5 109) (width 0.254) (layer "B.Cu") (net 7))
 (segment (start 144.5 109) (end 144 108.5) (width 0.254) (layer "B.Cu") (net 7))
 (segment (start 144 106.5) (end 144 108.5) (width 0.254) (layer "B.Cu") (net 7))
 (segment (start 143.422 108.022) (end 143.422 109.5095) (width 0.254) (layer "F.Cu") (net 3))
 (segment (start 143.422 109.5095) (end 144.4125 110.5) (width 0.254) (layer "F.Cu") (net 3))
 (segment (start 143.744 107.7) (end 143.422 108.022) (width 0.254) (layer "F.Cu") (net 3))
 (segment (start 143.7 107.7) (end 144 107.7) (width 0.254) (layer "F.Cu") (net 3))
 (segment (start 144 107.7) (end 143.744 107.7) (width 0.254) (layer "F.Cu") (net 3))
 (segment (start 140.5 104.5) (end 143.7 107.7) (width 0.254) (layer "F.Cu") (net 3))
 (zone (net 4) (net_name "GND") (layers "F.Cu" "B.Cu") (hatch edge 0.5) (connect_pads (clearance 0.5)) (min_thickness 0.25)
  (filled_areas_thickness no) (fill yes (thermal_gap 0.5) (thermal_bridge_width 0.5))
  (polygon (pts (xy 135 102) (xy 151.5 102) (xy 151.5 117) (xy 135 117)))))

